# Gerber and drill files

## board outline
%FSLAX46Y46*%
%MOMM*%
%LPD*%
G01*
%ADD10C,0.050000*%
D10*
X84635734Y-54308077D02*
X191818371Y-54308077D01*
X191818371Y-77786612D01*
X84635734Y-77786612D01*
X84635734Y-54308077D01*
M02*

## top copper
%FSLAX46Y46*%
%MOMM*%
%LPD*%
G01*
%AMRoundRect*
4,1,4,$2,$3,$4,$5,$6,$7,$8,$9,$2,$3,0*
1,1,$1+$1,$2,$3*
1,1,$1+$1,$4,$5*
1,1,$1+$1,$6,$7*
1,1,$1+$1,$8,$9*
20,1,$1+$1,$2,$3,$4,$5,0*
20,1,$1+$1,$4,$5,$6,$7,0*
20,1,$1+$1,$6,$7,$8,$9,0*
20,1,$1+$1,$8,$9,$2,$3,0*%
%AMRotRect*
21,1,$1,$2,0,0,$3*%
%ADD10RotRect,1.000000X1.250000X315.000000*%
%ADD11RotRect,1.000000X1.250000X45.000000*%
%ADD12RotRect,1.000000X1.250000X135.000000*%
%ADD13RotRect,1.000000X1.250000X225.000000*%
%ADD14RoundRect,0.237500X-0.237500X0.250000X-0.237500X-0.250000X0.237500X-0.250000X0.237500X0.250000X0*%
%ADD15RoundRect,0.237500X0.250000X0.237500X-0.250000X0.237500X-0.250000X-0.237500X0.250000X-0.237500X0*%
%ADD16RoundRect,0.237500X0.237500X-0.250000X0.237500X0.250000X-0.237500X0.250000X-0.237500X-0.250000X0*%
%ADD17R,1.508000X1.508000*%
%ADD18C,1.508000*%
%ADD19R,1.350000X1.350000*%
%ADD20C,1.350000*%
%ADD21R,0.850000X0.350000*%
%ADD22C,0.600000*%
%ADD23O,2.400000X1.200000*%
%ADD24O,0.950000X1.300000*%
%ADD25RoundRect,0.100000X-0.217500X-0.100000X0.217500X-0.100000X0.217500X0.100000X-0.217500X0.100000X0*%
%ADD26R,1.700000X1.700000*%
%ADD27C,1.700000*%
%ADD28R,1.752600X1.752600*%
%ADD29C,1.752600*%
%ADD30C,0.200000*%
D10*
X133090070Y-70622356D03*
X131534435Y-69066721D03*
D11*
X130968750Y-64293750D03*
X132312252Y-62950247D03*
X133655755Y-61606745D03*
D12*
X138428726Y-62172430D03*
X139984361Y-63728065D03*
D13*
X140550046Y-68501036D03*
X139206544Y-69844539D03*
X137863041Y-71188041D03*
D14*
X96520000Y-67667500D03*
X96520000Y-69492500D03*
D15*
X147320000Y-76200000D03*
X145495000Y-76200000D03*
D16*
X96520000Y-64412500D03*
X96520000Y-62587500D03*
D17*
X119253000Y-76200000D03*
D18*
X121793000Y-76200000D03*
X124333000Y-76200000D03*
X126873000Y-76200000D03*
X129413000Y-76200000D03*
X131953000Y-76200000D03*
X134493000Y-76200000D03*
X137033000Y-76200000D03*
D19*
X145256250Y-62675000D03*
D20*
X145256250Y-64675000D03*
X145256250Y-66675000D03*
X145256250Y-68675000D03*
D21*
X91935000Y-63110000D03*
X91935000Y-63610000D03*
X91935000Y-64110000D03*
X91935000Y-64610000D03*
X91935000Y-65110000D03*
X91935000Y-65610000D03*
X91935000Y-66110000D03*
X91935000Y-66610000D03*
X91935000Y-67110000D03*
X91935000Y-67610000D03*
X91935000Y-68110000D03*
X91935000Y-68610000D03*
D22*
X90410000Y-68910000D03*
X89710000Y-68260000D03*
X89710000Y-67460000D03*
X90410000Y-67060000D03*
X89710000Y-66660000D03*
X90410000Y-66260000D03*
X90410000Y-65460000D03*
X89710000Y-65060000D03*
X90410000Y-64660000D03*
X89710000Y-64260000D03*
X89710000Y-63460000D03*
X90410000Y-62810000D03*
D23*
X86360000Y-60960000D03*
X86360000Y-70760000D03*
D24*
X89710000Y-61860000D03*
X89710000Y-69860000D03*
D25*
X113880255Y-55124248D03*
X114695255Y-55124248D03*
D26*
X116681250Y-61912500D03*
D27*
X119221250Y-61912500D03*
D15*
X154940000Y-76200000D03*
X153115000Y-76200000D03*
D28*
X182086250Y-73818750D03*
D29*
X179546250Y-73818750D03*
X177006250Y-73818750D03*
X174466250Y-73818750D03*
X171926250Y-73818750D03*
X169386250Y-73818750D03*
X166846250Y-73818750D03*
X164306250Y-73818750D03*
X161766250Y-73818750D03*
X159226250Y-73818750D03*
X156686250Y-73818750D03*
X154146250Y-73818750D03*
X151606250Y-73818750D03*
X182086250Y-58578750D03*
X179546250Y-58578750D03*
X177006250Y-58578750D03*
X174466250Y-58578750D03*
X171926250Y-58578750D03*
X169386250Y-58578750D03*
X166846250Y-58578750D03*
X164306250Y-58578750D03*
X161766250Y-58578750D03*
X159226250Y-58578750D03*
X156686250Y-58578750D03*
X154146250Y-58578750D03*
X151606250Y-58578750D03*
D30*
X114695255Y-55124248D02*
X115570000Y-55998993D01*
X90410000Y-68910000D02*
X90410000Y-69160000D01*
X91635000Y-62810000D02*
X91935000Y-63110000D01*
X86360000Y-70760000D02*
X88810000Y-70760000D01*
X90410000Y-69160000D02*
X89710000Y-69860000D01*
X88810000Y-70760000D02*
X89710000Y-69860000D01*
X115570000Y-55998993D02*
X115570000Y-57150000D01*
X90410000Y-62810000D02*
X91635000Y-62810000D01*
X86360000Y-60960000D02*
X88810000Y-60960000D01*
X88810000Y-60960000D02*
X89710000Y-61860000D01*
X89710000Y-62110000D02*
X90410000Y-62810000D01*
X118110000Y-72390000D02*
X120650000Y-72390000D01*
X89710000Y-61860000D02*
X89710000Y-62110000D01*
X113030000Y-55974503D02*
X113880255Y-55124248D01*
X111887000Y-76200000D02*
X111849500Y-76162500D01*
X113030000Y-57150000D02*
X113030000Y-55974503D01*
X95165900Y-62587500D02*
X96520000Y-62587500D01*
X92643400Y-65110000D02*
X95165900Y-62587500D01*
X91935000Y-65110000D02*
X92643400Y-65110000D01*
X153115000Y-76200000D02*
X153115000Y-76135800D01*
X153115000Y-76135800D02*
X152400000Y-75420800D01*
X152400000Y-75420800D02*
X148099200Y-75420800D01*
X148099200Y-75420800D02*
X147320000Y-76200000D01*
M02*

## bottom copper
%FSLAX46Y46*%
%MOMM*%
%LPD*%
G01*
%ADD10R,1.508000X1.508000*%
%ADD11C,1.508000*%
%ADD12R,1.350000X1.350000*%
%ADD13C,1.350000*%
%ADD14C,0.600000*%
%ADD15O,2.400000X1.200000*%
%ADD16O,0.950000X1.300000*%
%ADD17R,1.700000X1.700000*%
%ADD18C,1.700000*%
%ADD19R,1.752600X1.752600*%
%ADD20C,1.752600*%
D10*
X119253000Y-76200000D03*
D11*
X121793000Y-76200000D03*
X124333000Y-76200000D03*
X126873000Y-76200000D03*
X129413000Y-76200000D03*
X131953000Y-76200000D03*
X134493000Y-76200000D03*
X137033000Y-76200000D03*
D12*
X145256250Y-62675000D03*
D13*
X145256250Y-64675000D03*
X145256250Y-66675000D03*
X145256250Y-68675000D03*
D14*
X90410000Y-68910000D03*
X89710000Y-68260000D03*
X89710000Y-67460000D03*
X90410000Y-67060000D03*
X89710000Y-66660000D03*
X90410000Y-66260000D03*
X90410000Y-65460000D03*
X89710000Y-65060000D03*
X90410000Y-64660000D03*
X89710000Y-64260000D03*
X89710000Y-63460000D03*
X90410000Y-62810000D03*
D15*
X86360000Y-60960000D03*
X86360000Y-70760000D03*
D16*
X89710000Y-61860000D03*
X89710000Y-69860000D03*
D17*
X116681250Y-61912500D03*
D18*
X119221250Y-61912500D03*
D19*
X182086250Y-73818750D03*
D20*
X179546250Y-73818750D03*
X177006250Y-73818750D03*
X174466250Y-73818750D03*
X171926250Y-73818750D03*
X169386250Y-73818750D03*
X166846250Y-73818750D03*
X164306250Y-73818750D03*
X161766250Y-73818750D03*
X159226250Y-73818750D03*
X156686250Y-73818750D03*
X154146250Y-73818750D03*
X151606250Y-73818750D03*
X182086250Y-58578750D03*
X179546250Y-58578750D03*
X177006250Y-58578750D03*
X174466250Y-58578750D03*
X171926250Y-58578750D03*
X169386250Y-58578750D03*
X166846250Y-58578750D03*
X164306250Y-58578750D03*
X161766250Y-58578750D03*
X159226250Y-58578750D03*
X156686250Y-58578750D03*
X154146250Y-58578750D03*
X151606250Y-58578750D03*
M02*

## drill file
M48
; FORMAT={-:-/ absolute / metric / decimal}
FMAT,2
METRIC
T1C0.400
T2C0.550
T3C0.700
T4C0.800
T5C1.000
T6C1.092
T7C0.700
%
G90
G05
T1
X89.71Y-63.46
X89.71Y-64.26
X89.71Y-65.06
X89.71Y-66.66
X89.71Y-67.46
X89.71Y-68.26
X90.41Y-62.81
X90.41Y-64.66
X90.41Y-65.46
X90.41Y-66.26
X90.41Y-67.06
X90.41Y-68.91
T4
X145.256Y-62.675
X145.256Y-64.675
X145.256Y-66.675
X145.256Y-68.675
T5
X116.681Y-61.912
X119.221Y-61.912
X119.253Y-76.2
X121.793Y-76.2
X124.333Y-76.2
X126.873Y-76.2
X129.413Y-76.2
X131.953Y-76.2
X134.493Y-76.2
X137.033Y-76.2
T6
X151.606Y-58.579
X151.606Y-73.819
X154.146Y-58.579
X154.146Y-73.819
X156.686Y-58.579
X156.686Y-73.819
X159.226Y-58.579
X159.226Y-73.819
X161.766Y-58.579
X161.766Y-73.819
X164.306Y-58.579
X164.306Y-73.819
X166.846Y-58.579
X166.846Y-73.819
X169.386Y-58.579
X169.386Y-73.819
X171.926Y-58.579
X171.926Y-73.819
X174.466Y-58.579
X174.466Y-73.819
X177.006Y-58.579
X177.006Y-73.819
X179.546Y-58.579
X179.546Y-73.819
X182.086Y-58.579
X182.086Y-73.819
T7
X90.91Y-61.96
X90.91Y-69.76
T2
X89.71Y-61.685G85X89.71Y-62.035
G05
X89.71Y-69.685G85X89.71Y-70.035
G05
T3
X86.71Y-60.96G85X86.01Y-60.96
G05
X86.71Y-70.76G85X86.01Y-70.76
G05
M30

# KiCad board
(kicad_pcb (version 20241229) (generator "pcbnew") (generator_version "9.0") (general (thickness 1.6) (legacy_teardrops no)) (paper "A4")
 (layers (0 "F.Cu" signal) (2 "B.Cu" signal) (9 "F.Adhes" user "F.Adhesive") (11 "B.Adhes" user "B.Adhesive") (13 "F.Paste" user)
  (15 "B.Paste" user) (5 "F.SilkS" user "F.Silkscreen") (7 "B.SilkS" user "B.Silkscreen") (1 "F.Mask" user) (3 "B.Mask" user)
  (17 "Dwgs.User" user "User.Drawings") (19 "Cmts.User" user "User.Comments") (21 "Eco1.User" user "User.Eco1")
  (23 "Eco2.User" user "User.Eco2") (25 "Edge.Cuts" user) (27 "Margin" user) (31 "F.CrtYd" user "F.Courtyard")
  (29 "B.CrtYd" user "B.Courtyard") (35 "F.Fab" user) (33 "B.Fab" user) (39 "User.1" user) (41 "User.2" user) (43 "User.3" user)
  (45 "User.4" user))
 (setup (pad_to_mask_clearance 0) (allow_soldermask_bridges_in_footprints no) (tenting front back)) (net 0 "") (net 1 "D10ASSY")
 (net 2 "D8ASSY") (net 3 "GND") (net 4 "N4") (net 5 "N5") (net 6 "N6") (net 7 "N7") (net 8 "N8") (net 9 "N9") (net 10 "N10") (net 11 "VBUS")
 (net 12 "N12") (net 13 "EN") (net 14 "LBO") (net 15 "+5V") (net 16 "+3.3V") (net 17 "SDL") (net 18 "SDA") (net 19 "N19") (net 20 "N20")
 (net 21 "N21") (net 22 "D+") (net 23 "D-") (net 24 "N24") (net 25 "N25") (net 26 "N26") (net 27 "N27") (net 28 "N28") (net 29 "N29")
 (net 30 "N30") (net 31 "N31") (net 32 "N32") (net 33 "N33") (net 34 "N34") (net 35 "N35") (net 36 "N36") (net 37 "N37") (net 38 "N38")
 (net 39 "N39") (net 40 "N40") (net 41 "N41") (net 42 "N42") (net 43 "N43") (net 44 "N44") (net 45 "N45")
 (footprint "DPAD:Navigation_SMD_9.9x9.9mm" (layer "F.Cu") (at 135.759398 66.397393 180)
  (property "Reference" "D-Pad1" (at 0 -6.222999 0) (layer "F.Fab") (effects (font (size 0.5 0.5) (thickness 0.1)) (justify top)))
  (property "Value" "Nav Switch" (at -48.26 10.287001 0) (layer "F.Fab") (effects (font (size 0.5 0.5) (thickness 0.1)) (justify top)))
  (pad "1" smd rect (at 2.669328 -4.224963 315) (size 1 1.25) (layers "F.Cu" "F.Mask" "F.Paste") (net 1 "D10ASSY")
   (solder_mask_margin 0.1016) (thermal_bridge_angle 0))
  (pad "2" smd rect (at 4.224963 -2.669328 315) (size 1 1.25) (layers "F.Cu" "F.Mask" "F.Paste") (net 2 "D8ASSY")
   (solder_mask_margin 0.1016) (thermal_bridge_angle 0))
  (pad "3" smd rect (at 4.790648 2.103643 45) (size 1 1.25) (layers "F.Cu" "F.Mask" "F.Paste") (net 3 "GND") (solder_mask_margin 0.1016)
   (thermal_bridge_angle 0))
  (pad "4" smd rect (at 3.447146 3.447146 45) (size 1 1.25) (layers "F.Cu" "F.Mask" "F.Paste") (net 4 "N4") (solder_mask_margin 0.1016)
   (thermal_bridge_angle 0))
  (pad "5" smd rect (at 2.103643 4.790648 45) (size 1 1.25) (layers "F.Cu" "F.Mask" "F.Paste") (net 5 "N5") (solder_mask_margin 0.1016)
   (thermal_bridge_angle 0))
  (pad "6" smd rect (at -2.669328 4.224963 135) (size 1 1.25) (layers "F.Cu" "F.Mask" "F.Paste") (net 3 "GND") (solder_mask_margin 0.1016)
   (thermal_bridge_angle 0))
  (pad "7" smd rect (at -4.224963 2.669328 135) (size 1 1.25) (layers "F.Cu" "F.Mask" "F.Paste") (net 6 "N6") (solder_mask_margin 0.1016)
   (thermal_bridge_angle 0))
  (pad "8" smd rect (at -4.790648 -2.103643 225) (size 1 1.25) (layers "F.Cu" "F.Mask" "F.Paste") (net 3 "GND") (solder_mask_margin 0.1016)
   (thermal_bridge_angle 0))
  (pad "9" smd rect (at -3.447146 -3.447146 225) (size 1 1.25) (layers "F.Cu" "F.Mask" "F.Paste") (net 3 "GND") (solder_mask_margin 0.1016)
   (thermal_bridge_angle 0))
  (pad "10" smd rect (at -2.103643 -4.790648 225) (size 1 1.25) (layers "F.Cu" "F.Mask" "F.Paste") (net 3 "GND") (solder_mask_margin 0.1016)
   (thermal_bridge_angle 0)))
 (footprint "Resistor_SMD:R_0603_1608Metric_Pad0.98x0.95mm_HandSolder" (layer "F.Cu") (at 96.52 68.58 -90)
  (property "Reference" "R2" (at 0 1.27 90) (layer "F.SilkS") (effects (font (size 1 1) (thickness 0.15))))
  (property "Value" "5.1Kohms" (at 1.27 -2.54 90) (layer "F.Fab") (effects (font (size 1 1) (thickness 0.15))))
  (pad "1" smd roundrect (at -0.9125 0 270) (size 0.975 0.95) (layers "F.Cu" "F.Mask" "F.Paste") (roundrect_rratio 0.25) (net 3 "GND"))
  (pad "2" smd roundrect (at 0.9125 0 270) (size 0.975 0.95) (layers "F.Cu" "F.Mask" "F.Paste") (roundrect_rratio 0.25) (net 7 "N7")))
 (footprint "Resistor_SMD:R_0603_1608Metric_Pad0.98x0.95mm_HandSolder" (layer "F.Cu") (at 146.4075 76.2 180)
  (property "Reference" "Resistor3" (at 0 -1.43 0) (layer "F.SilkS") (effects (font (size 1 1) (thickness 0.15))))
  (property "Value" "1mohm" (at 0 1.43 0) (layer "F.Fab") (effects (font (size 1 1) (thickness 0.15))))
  (pad "1" smd roundrect (at -0.9125 0 180) (size 0.975 0.95) (layers "F.Cu" "F.Mask" "F.Paste") (roundrect_rratio 0.25) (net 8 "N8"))
  (pad "2" smd roundrect (at 0.9125 0 180) (size 0.975 0.95) (layers "F.Cu" "F.Mask" "F.Paste") (roundrect_rratio 0.25) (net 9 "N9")))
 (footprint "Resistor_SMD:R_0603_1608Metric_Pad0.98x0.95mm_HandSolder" (layer "F.Cu") (at 96.52 63.5 90)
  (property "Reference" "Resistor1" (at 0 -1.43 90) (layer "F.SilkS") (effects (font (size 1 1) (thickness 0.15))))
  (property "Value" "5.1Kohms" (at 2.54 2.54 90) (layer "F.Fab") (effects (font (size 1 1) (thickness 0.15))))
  (pad "1" smd roundrect (at -0.9125 0 90) (size 0.975 0.95) (layers "F.Cu" "F.Mask" "F.Paste") (roundrect_rratio 0.25) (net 3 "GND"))
  (pad "2" smd roundrect (at 0.9125 0 90) (size 0.975 0.95) (layers "F.Cu" "F.Mask" "F.Paste") (roundrect_rratio 0.25) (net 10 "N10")))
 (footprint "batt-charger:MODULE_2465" (layer "F.Cu") (at 124.46 66.04)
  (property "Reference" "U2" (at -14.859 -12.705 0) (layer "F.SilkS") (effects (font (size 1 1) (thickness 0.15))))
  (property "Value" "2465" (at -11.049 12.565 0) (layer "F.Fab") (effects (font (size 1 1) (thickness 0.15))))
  (pad "1" thru_hole rect (at -5.207 10.16) (size 1.508 1.508) (drill 1) (layers "*.Cu" "*.Mask") (remove_unused_layers no) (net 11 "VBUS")
   (solder_mask_margin 0.102))
  (pad "2" thru_hole circle (at -2.667 10.16) (size 1.508 1.508) (drill 1) (layers "*.Cu" "*.Mask") (remove_unused_layers no) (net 9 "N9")
   (solder_mask_margin 0.102))
  (pad "3" thru_hole circle (at -0.127 10.16) (size 1.508 1.508) (drill 1) (layers "*.Cu" "*.Mask") (remove_unused_layers no) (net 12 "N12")
   (solder_mask_margin 0.102))
  (pad "4" thru_hole circle (at 2.413 10.16) (size 1.508 1.508) (drill 1) (layers "*.Cu" "*.Mask") (remove_unused_layers no) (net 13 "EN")
   (solder_mask_margin 0.102))
  (pad "5" thru_hole circle (at 4.953 10.16) (size 1.508 1.508) (drill 1) (layers "*.Cu" "*.Mask") (remove_unused_layers no) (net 3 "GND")
   (solder_mask_margin 0.102))
  (pad "6" thru_hole circle (at 7.493 10.16) (size 1.508 1.508) (drill 1) (layers "*.Cu" "*.Mask") (remove_unused_layers no) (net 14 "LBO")
   (solder_mask_margin 0.102))
  (pad "7" thru_hole circle (at 10.033 10.16) (size 1.508 1.508) (drill 1) (layers "*.Cu" "*.Mask") (remove_unused_layers no) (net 3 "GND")
   (solder_mask_margin 0.102))
  (pad "8" thru_hole circle (at 12.573 10.16) (size 1.508 1.508) (drill 1) (layers "*.Cu" "*.Mask") (remove_unused_layers no) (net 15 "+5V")
   (solder_mask_margin 0.102)))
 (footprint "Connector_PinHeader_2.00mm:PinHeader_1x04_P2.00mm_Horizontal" (layer "F.Cu") (at 145.25625 62.675)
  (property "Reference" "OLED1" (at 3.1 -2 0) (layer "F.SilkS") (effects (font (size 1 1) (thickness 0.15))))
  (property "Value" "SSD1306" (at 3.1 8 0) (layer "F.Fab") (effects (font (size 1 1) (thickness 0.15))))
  (pad "1" thru_hole rect (at 0 0) (size 1.35 1.35) (drill 0.8) (layers "*.Cu" "*.Mask") (remove_unused_layers no) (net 3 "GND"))
  (pad "2" thru_hole circle (at 0 2) (size 1.35 1.35) (drill 0.8) (layers "*.Cu" "*.Mask") (remove_unused_layers no) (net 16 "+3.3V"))
  (pad "3" thru_hole circle (at 0 4) (size 1.35 1.35) (drill 0.8) (layers "*.Cu" "*.Mask") (remove_unused_layers no) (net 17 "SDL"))
  (pad "4" thru_hole circle (at 0 6) (size 1.35 1.35) (drill 0.8) (layers "*.Cu" "*.Mask") (remove_unused_layers no) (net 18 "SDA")))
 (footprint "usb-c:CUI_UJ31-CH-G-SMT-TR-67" (layer "F.Cu") (at 86.36 65.86 -90)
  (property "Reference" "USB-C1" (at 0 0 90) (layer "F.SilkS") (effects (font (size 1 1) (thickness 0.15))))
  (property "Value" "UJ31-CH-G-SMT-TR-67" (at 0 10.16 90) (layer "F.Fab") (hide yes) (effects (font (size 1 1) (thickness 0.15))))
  (pad "" np_thru_hole circle (at -3.9 -4.55 270) (size 0.7 0.7) (drill 0.7) (layers "*.Cu" "*.Mask"))
  (pad "" np_thru_hole circle (at 3.9 -4.55 270) (size 0.7 0.7) (drill 0.7) (layers "*.Cu" "*.Mask"))
  (pad "A1" smd rect (at -2.75 -5.575 270) (size 0.35 0.85) (layers "F.Cu" "F.Mask" "F.Paste") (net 3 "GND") (solder_mask_margin 0.102))
  (pad "A2" smd rect (at -2.25 -5.575 270) (size 0.35 0.85) (layers "F.Cu" "F.Mask" "F.Paste") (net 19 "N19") (solder_mask_margin 0.102))
  (pad "A3" smd rect (at -1.75 -5.575 270) (size 0.35 0.85) (layers "F.Cu" "F.Mask" "F.Paste") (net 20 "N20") (solder_mask_margin 0.102))
  (pad "A4" smd rect (at -1.25 -5.575 270) (size 0.35 0.85) (layers "F.Cu" "F.Mask" "F.Paste") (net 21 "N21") (solder_mask_margin 0.102))
  (pad "A5" smd rect (at -0.75 -5.575 270) (size 0.35 0.85) (layers "F.Cu" "F.Mask" "F.Paste") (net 10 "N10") (solder_mask_margin 0.102))
  (pad "A6" smd rect (at -0.25 -5.575 270) (size 0.35 0.85) (layers "F.Cu" "F.Mask" "F.Paste") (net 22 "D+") (solder_mask_margin 0.102))
  (pad "A7" smd rect (at 0.25 -5.575 270) (size 0.35 0.85) (layers "F.Cu" "F.Mask" "F.Paste") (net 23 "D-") (solder_mask_margin 0.102))
  (pad "A8" smd rect (at 0.75 -5.575 270) (size 0.35 0.85) (layers "F.Cu" "F.Mask" "F.Paste") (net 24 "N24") (solder_mask_margin 0.102))
  (pad "A9" smd rect (at 1.25 -5.575 270) (size 0.35 0.85) (layers "F.Cu" "F.Mask" "F.Paste") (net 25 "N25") (solder_mask_margin 0.102))
  (pad "A10" smd rect (at 1.75 -5.575 270) (size 0.35 0.85) (layers "F.Cu" "F.Mask" "F.Paste") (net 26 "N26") (solder_mask_margin 0.102))
  (pad "A11" smd rect (at 2.25 -5.575 270) (size 0.35 0.85) (layers "F.Cu" "F.Mask" "F.Paste") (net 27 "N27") (solder_mask_margin 0.102))
  (pad "A12" smd rect (at 2.75 -5.575 270) (size 0.35 0.85) (layers "F.Cu" "F.Mask" "F.Paste") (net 3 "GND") (solder_mask_margin 0.102))
  (pad "B1" thru_hole circle (at 3.05 -4.05 270) (size 0.6 0.6) (drill 0.4) (layers "*.Cu" "*.Mask") (remove_unused_layers no) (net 3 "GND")
   (solder_mask_margin 0.102))
  (pad "B2" thru_hole circle (at 2.4 -3.35 270) (size 0.6 0.6) (drill 0.4) (layers "*.Cu" "*.Mask") (remove_unused_layers no) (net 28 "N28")
   (solder_mask_margin 0.102))
  (pad "B3" thru_hole circle (at 1.6 -3.35 270) (size 0.6 0.6) (drill 0.4) (layers "*.Cu" "*.Mask") (remove_unused_layers no) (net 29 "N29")
   (solder_mask_margin 0.102))
  (pad "B4" thru_hole circle (at 1.2 -4.05 270) (size 0.6 0.6) (drill 0.4) (layers "*.Cu" "*.Mask") (remove_unused_layers no) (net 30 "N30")
   (solder_mask_margin 0.102))
  (pad "B5" thru_hole circle (at 0.8 -3.35 270) (size 0.6 0.6) (drill 0.4) (layers "*.Cu" "*.Mask") (remove_unused_layers no) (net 7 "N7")
   (solder_mask_margin 0.102))
  (pad "B6" thru_hole circle (at 0.4 -4.05 270) (size 0.6 0.6) (drill 0.4) (layers "*.Cu" "*.Mask") (remove_unused_layers no) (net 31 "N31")
   (solder_mask_margin 0.102))
  (pad "B7" thru_hole circle (at -0.4 -4.05 270) (size 0.6 0.6) (drill 0.4) (layers "*.Cu" "*.Mask") (remove_unused_layers no)
   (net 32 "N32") (solder_mask_margin 0.102))
  (pad "B8" thru_hole circle (at -0.8 -3.35 270) (size 0.6 0.6) (drill 0.4) (layers "*.Cu" "*.Mask") (remove_unused_layers no)
   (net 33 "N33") (solder_mask_margin 0.102))
  (pad "B9" thru_hole circle (at -1.2 -4.05 270) (size 0.6 0.6) (drill 0.4) (layers "*.Cu" "*.Mask") (remove_unused_layers no)
   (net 11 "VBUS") (solder_mask_margin 0.102))
  (pad "B10" thru_hole circle (at -1.6 -3.35 270) (size 0.6 0.6) (drill 0.4) (layers "*.Cu" "*.Mask") (remove_unused_layers no)
   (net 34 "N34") (solder_mask_margin 0.102))
  (pad "B11" thru_hole circle (at -2.4 -3.35 270) (size 0.6 0.6) (drill 0.4) (layers "*.Cu" "*.Mask") (remove_unused_layers no)
   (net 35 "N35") (solder_mask_margin 0.102))
  (pad "B12" thru_hole circle (at -3.05 -4.05 270) (size 0.6 0.6) (drill 0.4) (layers "*.Cu" "*.Mask") (remove_unused_layers no)
   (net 3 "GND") (solder_mask_margin 0.102))
  (pad "S1" thru_hole oval (at -4.9 0 270) (size 1.2 2.4) (drill oval 0.7 1.4) (layers "*.Cu" "*.Mask") (remove_unused_layers no)
   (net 3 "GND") (solder_mask_margin 0.102))
  (pad "S2" thru_hole oval (at 4.9 0 270) (size 1.2 2.4) (drill oval 0.7 1.4) (layers "*.Cu" "*.Mask") (remove_unused_layers no)
   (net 3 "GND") (solder_mask_margin 0.102))
  (pad "S3" thru_hole oval (at -4 -3.35 270) (size 1.3 0.95) (drill oval 0.9 0.55) (layers "*.Cu" "*.Mask") (remove_unused_layers no)
   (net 3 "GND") (solder_mask_margin 0.102))
  (pad "S4" thru_hole oval (at 4 -3.35 270) (size 1.3 0.95) (drill oval 0.9 0.55) (layers "*.Cu" "*.Mask") (remove_unused_layers no)
   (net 3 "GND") (solder_mask_margin 0.102)))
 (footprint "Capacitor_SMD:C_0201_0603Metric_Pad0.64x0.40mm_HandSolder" (layer "F.Cu") (at 114.287755 55.124248)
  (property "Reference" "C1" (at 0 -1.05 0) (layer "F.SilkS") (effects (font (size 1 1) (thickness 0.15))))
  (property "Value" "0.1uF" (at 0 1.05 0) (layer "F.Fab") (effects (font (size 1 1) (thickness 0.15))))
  (pad "" smd roundrect (at -0.4325 0) (size 0.458 0.36) (layers "F.Paste") (roundrect_rratio 0.25))
  (pad "" smd roundrect (at 0.4325 0) (size 0.458 0.36) (layers "F.Paste") (roundrect_rratio 0.25))
  (pad "1" smd roundrect (at -0.4075 0) (size 0.635 0.4) (layers "F.Cu" "F.Mask") (roundrect_rratio 0.25) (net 15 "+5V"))
  (pad "2" smd roundrect (at 0.4075 0) (size 0.635 0.4) (layers "F.Cu" "F.Mask") (roundrect_rratio 0.25) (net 3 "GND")))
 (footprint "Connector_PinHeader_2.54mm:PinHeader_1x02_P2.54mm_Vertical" (layer "F.Cu") (at 116.68125 61.9125 90)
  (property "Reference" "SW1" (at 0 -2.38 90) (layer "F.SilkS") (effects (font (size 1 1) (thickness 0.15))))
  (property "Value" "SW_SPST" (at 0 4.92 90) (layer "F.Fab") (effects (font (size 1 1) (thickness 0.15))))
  (pad "1" thru_hole rect (at 0 0 90) (size 1.7 1.7) (drill 1) (layers "*.Cu" "*.Mask") (remove_unused_layers no) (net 13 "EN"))
  (pad "2" thru_hole circle (at 0 2.54 90) (size 1.7 1.7) (drill 1) (layers "*.Cu" "*.Mask") (remove_unused_layers no) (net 3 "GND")))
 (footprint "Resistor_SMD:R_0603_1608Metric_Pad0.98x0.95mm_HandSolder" (layer "F.Cu") (at 154.0275 76.2 180)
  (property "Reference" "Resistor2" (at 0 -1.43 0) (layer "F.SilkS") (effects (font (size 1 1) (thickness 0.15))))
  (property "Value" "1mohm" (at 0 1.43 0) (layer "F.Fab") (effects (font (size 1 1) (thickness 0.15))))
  (pad "1" smd roundrect (at -0.9125 0 180) (size 0.975 0.95) (layers "F.Cu" "F.Mask" "F.Paste") (roundrect_rratio 0.25) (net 3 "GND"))
  (pad "2" smd roundrect (at 0.9125 0 180) (size 0.975 0.95) (layers "F.Cu" "F.Mask" "F.Paste") (roundrect_rratio 0.25) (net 8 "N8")))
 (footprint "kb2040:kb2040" (layer "B.Cu") (at 168.11625 66.19875 90)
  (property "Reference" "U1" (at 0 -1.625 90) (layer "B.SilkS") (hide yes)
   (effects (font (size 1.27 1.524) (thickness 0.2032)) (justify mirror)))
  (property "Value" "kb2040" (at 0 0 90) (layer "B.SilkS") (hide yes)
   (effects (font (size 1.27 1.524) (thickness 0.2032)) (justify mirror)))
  (pad "1" thru_hole rect (at -7.62 13.97 180) (size 1.7526 1.7526) (drill 1.0922) (layers "*.Cu" "*.SilkS" "*.Mask")
   (remove_unused_layers no) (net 22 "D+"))
  (pad "2" thru_hole circle (at -7.62 11.43 180) (size 1.7526 1.7526) (drill 1.0922) (layers "*.Cu" "*.SilkS" "*.Mask")
   (remove_unused_layers no) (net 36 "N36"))
  (pad "3" thru_hole circle (at -7.62 8.89 180) (size 1.7526 1.7526) (drill 1.0922) (layers "*.Cu" "*.SilkS" "*.Mask")
   (remove_unused_layers no) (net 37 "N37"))
  (pad "4" thru_hole circle (at -7.62 6.35 180) (size 1.7526 1.7526) (drill 1.0922) (layers "*.Cu" "*.SilkS" "*.Mask")
   (remove_unused_layers no) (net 3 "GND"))
  (pad "5" thru_hole circle (at -7.62 3.81 180) (size 1.7526 1.7526) (drill 1.0922) (layers "*.Cu" "*.SilkS" "*.Mask")
   (remove_unused_layers no) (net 3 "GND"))
  (pad "6" thru_hole circle (at -7.62 1.27 180) (size 1.7526 1.7526) (drill 1.0922) (layers "*.Cu" "*.SilkS" "*.Mask")
   (remove_unused_layers no) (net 17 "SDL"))
  (pad "7" thru_hole circle (at -7.62 -1.27 180) (size 1.7526 1.7526) (drill 1.0922) (layers "*.Cu" "*.SilkS" "*.Mask")
   (remove_unused_layers no) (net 18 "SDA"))
  (pad "8" thru_hole circle (at -7.62 -3.81 180) (size 1.7526 1.7526) (drill 1.0922) (layers "*.Cu" "*.SilkS" "*.Mask")
   (remove_unused_layers no) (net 2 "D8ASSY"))
  (pad "9" thru_hole circle (at -7.62 -6.35 180) (size 1.7526 1.7526) (drill 1.0922) (layers "*.Cu" "*.SilkS" "*.Mask")
   (remove_unused_layers no) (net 4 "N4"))
  (pad "10" thru_hole circle (at -7.62 -8.89 180) (size 1.7526 1.7526) (drill 1.0922) (layers "*.Cu" "*.SilkS" "*.Mask")
   (remove_unused_layers no) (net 1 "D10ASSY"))
  (pad "11" thru_hole circle (at -7.62 -11.43 180) (size 1.7526 1.7526) (drill 1.0922) (layers "*.Cu" "*.SilkS" "*.Mask")
   (remove_unused_layers no) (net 5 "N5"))
  (pad "12" thru_hole circle (at -7.62 -13.97 180) (size 1.7526 1.7526) (drill 1.0922) (layers "*.Cu" "*.SilkS" "*.Mask")
   (remove_unused_layers no) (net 6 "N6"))
  (pad "13" thru_hole circle (at -7.62 -16.51 180) (size 1.7526 1.7526) (drill 1.0922) (layers "*.Cu" "*.SilkS" "*.Mask")
   (remove_unused_layers no) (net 14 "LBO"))
  (pad "14" thru_hole circle (at 7.62 13.97 180) (size 1.7526 1.7526) (drill 1.0922) (layers "*.Cu" "*.SilkS" "*.Mask")
   (remove_unused_layers no) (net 23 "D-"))
  (pad "15" thru_hole circle (at 7.62 11.43 180) (size 1.7526 1.7526) (drill 1.0922) (layers "*.Cu" "*.SilkS" "*.Mask")
   (remove_unused_layers no) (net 15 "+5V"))
  (pad "16" thru_hole circle (at 7.62 8.89 180) (size 1.7526 1.7526) (drill 1.0922) (layers "*.Cu" "*.SilkS" "*.Mask")
   (remove_unused_layers no) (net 3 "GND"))
  (pad "17" thru_hole circle (at 7.62 6.35 180) (size 1.7526 1.7526) (drill 1.0922) (layers "*.Cu" "*.SilkS" "*.Mask")
   (remove_unused_layers no) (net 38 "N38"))
  (pad "18" thru_hole circle (at 7.62 3.81 180) (size 1.7526 1.7526) (drill 1.0922) (layers "*.Cu" "*.SilkS" "*.Mask")
   (remove_unused_layers no) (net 16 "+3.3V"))
  (pad "19" thru_hole circle (at 7.62 1.27 180) (size 1.7526 1.7526) (drill 1.0922) (layers "*.Cu" "*.SilkS" "*.Mask")
   (remove_unused_layers no) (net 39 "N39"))
  (pad "20" thru_hole circle (at 7.62 -1.27 180) (size 1.7526 1.7526) (drill 1.0922) (layers "*.Cu" "*.SilkS" "*.Mask")
   (remove_unused_layers no) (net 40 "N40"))
  (pad "21" thru_hole circle (at 7.62 -3.81 180) (size 1.7526 1.7526) (drill 1.0922) (layers "*.Cu" "*.SilkS" "*.Mask")
   (remove_unused_layers no) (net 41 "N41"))
  (pad "22" thru_hole circle (at 7.62 -6.35 180) (size 1.7526 1.7526) (drill 1.0922) (layers "*.Cu" "*.SilkS" "*.Mask")
   (remove_unused_layers no) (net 8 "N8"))
  (pad "23" thru_hole circle (at 7.62 -8.89 180) (size 1.7526 1.7526) (drill 1.0922) (layers "*.Cu" "*.SilkS" "*.Mask")
   (remove_unused_layers no) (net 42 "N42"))
  (pad "24" thru_hole circle (at 7.62 -11.43 180) (size 1.7526 1.7526) (drill 1.0922) (layers "*.Cu" "*.SilkS" "*.Mask")
   (remove_unused_layers no) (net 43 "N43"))
  (pad "25" thru_hole circle (at 7.62 -13.97 180) (size 1.7526 1.7526) (drill 1.0922) (layers "*.Cu" "*.SilkS" "*.Mask")
   (remove_unused_layers no) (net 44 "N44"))
  (pad "26" thru_hole circle (at 7.62 -16.51 180) (size 1.7526 1.7526) (drill 1.0922) (layers "*.Cu" "*.SilkS" "*.Mask")
   (remove_unused_layers no) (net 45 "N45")))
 (gr_rect (start 84.635734 54.308077) (end 191.818371 77.786612) (stroke (width 0.05) (type default)) (fill no) (layer "Edge.Cuts"))
 (segment (start 114.695255 55.124248) (end 115.57 55.998993) (width 0.2) (layer "F.Cu") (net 3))
 (segment (start 90.41 68.91) (end 90.41 69.16) (width 0.2) (layer "F.Cu") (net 3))
 (segment (start 91.635 62.81) (end 91.935 63.11) (width 0.2) (layer "F.Cu") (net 3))
 (segment (start 86.36 70.76) (end 88.81 70.76) (width 0.2) (layer "F.Cu") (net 3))
 (segment (start 90.41 69.16) (end 89.71 69.86) (width 0.2) (layer "F.Cu") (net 3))
 (segment (start 88.81 70.76) (end 89.71 69.86) (width 0.2) (layer "F.Cu") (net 3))
 (segment (start 115.57 55.998993) (end 115.57 57.15) (width 0.2) (layer "F.Cu") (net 3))
 (segment (start 90.41 62.81) (end 91.635 62.81) (width 0.2) (layer "F.Cu") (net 3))
 (segment (start 86.36 60.96) (end 88.81 60.96) (width 0.2) (layer "F.Cu") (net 3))
 (segment (start 88.81 60.96) (end 89.71 61.86) (width 0.2) (layer "F.Cu") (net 3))
 (segment (start 89.71 62.11) (end 90.41 62.81) (width 0.2) (layer "F.Cu") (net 3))
 (segment (start 118.11 72.39) (end 120.65 72.39) (width 0.2) (layer "F.Cu") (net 3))
 (segment (start 89.71 61.86) (end 89.71 62.11) (width 0.2) (layer "F.Cu") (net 3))
 (segment (start 113.03 55.974503) (end 113.880255 55.124248) (width 0.2) (layer "F.Cu") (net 15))
 (segment (start 111.887 76.2) (end 111.8495 76.1625) (width 0.2) (layer "F.Cu") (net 15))
 (segment (start 113.03 57.15) (end 113.03 55.974503) (width 0.2) (layer "F.Cu") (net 15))
 (segment (start 95.1659 62.5875) (end 96.52 62.5875) (width 0.2) (layer "F.Cu") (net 10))
 (segment (start 92.6434 65.11) (end 95.1659 62.5875) (width 0.2) (layer "F.Cu") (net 10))
 (segment (start 91.935 65.11) (end 92.6434 65.11) (width 0.2) (layer "F.Cu") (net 10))
 (segment (start 153.115 76.2) (end 153.115 76.1358) (width 0.2) (layer "F.Cu") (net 8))
 (segment (start 153.115 76.1358) (end 152.4 75.4208) (width 0.2) (layer "F.Cu") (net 8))
 (segment (start 152.4 75.4208) (end 148.0992 75.4208) (width 0.2) (layer "F.Cu") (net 8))
 (segment (start 148.0992 75.4208) (end 147.32 76.2) (width 0.2) (layer "F.Cu") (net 8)))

